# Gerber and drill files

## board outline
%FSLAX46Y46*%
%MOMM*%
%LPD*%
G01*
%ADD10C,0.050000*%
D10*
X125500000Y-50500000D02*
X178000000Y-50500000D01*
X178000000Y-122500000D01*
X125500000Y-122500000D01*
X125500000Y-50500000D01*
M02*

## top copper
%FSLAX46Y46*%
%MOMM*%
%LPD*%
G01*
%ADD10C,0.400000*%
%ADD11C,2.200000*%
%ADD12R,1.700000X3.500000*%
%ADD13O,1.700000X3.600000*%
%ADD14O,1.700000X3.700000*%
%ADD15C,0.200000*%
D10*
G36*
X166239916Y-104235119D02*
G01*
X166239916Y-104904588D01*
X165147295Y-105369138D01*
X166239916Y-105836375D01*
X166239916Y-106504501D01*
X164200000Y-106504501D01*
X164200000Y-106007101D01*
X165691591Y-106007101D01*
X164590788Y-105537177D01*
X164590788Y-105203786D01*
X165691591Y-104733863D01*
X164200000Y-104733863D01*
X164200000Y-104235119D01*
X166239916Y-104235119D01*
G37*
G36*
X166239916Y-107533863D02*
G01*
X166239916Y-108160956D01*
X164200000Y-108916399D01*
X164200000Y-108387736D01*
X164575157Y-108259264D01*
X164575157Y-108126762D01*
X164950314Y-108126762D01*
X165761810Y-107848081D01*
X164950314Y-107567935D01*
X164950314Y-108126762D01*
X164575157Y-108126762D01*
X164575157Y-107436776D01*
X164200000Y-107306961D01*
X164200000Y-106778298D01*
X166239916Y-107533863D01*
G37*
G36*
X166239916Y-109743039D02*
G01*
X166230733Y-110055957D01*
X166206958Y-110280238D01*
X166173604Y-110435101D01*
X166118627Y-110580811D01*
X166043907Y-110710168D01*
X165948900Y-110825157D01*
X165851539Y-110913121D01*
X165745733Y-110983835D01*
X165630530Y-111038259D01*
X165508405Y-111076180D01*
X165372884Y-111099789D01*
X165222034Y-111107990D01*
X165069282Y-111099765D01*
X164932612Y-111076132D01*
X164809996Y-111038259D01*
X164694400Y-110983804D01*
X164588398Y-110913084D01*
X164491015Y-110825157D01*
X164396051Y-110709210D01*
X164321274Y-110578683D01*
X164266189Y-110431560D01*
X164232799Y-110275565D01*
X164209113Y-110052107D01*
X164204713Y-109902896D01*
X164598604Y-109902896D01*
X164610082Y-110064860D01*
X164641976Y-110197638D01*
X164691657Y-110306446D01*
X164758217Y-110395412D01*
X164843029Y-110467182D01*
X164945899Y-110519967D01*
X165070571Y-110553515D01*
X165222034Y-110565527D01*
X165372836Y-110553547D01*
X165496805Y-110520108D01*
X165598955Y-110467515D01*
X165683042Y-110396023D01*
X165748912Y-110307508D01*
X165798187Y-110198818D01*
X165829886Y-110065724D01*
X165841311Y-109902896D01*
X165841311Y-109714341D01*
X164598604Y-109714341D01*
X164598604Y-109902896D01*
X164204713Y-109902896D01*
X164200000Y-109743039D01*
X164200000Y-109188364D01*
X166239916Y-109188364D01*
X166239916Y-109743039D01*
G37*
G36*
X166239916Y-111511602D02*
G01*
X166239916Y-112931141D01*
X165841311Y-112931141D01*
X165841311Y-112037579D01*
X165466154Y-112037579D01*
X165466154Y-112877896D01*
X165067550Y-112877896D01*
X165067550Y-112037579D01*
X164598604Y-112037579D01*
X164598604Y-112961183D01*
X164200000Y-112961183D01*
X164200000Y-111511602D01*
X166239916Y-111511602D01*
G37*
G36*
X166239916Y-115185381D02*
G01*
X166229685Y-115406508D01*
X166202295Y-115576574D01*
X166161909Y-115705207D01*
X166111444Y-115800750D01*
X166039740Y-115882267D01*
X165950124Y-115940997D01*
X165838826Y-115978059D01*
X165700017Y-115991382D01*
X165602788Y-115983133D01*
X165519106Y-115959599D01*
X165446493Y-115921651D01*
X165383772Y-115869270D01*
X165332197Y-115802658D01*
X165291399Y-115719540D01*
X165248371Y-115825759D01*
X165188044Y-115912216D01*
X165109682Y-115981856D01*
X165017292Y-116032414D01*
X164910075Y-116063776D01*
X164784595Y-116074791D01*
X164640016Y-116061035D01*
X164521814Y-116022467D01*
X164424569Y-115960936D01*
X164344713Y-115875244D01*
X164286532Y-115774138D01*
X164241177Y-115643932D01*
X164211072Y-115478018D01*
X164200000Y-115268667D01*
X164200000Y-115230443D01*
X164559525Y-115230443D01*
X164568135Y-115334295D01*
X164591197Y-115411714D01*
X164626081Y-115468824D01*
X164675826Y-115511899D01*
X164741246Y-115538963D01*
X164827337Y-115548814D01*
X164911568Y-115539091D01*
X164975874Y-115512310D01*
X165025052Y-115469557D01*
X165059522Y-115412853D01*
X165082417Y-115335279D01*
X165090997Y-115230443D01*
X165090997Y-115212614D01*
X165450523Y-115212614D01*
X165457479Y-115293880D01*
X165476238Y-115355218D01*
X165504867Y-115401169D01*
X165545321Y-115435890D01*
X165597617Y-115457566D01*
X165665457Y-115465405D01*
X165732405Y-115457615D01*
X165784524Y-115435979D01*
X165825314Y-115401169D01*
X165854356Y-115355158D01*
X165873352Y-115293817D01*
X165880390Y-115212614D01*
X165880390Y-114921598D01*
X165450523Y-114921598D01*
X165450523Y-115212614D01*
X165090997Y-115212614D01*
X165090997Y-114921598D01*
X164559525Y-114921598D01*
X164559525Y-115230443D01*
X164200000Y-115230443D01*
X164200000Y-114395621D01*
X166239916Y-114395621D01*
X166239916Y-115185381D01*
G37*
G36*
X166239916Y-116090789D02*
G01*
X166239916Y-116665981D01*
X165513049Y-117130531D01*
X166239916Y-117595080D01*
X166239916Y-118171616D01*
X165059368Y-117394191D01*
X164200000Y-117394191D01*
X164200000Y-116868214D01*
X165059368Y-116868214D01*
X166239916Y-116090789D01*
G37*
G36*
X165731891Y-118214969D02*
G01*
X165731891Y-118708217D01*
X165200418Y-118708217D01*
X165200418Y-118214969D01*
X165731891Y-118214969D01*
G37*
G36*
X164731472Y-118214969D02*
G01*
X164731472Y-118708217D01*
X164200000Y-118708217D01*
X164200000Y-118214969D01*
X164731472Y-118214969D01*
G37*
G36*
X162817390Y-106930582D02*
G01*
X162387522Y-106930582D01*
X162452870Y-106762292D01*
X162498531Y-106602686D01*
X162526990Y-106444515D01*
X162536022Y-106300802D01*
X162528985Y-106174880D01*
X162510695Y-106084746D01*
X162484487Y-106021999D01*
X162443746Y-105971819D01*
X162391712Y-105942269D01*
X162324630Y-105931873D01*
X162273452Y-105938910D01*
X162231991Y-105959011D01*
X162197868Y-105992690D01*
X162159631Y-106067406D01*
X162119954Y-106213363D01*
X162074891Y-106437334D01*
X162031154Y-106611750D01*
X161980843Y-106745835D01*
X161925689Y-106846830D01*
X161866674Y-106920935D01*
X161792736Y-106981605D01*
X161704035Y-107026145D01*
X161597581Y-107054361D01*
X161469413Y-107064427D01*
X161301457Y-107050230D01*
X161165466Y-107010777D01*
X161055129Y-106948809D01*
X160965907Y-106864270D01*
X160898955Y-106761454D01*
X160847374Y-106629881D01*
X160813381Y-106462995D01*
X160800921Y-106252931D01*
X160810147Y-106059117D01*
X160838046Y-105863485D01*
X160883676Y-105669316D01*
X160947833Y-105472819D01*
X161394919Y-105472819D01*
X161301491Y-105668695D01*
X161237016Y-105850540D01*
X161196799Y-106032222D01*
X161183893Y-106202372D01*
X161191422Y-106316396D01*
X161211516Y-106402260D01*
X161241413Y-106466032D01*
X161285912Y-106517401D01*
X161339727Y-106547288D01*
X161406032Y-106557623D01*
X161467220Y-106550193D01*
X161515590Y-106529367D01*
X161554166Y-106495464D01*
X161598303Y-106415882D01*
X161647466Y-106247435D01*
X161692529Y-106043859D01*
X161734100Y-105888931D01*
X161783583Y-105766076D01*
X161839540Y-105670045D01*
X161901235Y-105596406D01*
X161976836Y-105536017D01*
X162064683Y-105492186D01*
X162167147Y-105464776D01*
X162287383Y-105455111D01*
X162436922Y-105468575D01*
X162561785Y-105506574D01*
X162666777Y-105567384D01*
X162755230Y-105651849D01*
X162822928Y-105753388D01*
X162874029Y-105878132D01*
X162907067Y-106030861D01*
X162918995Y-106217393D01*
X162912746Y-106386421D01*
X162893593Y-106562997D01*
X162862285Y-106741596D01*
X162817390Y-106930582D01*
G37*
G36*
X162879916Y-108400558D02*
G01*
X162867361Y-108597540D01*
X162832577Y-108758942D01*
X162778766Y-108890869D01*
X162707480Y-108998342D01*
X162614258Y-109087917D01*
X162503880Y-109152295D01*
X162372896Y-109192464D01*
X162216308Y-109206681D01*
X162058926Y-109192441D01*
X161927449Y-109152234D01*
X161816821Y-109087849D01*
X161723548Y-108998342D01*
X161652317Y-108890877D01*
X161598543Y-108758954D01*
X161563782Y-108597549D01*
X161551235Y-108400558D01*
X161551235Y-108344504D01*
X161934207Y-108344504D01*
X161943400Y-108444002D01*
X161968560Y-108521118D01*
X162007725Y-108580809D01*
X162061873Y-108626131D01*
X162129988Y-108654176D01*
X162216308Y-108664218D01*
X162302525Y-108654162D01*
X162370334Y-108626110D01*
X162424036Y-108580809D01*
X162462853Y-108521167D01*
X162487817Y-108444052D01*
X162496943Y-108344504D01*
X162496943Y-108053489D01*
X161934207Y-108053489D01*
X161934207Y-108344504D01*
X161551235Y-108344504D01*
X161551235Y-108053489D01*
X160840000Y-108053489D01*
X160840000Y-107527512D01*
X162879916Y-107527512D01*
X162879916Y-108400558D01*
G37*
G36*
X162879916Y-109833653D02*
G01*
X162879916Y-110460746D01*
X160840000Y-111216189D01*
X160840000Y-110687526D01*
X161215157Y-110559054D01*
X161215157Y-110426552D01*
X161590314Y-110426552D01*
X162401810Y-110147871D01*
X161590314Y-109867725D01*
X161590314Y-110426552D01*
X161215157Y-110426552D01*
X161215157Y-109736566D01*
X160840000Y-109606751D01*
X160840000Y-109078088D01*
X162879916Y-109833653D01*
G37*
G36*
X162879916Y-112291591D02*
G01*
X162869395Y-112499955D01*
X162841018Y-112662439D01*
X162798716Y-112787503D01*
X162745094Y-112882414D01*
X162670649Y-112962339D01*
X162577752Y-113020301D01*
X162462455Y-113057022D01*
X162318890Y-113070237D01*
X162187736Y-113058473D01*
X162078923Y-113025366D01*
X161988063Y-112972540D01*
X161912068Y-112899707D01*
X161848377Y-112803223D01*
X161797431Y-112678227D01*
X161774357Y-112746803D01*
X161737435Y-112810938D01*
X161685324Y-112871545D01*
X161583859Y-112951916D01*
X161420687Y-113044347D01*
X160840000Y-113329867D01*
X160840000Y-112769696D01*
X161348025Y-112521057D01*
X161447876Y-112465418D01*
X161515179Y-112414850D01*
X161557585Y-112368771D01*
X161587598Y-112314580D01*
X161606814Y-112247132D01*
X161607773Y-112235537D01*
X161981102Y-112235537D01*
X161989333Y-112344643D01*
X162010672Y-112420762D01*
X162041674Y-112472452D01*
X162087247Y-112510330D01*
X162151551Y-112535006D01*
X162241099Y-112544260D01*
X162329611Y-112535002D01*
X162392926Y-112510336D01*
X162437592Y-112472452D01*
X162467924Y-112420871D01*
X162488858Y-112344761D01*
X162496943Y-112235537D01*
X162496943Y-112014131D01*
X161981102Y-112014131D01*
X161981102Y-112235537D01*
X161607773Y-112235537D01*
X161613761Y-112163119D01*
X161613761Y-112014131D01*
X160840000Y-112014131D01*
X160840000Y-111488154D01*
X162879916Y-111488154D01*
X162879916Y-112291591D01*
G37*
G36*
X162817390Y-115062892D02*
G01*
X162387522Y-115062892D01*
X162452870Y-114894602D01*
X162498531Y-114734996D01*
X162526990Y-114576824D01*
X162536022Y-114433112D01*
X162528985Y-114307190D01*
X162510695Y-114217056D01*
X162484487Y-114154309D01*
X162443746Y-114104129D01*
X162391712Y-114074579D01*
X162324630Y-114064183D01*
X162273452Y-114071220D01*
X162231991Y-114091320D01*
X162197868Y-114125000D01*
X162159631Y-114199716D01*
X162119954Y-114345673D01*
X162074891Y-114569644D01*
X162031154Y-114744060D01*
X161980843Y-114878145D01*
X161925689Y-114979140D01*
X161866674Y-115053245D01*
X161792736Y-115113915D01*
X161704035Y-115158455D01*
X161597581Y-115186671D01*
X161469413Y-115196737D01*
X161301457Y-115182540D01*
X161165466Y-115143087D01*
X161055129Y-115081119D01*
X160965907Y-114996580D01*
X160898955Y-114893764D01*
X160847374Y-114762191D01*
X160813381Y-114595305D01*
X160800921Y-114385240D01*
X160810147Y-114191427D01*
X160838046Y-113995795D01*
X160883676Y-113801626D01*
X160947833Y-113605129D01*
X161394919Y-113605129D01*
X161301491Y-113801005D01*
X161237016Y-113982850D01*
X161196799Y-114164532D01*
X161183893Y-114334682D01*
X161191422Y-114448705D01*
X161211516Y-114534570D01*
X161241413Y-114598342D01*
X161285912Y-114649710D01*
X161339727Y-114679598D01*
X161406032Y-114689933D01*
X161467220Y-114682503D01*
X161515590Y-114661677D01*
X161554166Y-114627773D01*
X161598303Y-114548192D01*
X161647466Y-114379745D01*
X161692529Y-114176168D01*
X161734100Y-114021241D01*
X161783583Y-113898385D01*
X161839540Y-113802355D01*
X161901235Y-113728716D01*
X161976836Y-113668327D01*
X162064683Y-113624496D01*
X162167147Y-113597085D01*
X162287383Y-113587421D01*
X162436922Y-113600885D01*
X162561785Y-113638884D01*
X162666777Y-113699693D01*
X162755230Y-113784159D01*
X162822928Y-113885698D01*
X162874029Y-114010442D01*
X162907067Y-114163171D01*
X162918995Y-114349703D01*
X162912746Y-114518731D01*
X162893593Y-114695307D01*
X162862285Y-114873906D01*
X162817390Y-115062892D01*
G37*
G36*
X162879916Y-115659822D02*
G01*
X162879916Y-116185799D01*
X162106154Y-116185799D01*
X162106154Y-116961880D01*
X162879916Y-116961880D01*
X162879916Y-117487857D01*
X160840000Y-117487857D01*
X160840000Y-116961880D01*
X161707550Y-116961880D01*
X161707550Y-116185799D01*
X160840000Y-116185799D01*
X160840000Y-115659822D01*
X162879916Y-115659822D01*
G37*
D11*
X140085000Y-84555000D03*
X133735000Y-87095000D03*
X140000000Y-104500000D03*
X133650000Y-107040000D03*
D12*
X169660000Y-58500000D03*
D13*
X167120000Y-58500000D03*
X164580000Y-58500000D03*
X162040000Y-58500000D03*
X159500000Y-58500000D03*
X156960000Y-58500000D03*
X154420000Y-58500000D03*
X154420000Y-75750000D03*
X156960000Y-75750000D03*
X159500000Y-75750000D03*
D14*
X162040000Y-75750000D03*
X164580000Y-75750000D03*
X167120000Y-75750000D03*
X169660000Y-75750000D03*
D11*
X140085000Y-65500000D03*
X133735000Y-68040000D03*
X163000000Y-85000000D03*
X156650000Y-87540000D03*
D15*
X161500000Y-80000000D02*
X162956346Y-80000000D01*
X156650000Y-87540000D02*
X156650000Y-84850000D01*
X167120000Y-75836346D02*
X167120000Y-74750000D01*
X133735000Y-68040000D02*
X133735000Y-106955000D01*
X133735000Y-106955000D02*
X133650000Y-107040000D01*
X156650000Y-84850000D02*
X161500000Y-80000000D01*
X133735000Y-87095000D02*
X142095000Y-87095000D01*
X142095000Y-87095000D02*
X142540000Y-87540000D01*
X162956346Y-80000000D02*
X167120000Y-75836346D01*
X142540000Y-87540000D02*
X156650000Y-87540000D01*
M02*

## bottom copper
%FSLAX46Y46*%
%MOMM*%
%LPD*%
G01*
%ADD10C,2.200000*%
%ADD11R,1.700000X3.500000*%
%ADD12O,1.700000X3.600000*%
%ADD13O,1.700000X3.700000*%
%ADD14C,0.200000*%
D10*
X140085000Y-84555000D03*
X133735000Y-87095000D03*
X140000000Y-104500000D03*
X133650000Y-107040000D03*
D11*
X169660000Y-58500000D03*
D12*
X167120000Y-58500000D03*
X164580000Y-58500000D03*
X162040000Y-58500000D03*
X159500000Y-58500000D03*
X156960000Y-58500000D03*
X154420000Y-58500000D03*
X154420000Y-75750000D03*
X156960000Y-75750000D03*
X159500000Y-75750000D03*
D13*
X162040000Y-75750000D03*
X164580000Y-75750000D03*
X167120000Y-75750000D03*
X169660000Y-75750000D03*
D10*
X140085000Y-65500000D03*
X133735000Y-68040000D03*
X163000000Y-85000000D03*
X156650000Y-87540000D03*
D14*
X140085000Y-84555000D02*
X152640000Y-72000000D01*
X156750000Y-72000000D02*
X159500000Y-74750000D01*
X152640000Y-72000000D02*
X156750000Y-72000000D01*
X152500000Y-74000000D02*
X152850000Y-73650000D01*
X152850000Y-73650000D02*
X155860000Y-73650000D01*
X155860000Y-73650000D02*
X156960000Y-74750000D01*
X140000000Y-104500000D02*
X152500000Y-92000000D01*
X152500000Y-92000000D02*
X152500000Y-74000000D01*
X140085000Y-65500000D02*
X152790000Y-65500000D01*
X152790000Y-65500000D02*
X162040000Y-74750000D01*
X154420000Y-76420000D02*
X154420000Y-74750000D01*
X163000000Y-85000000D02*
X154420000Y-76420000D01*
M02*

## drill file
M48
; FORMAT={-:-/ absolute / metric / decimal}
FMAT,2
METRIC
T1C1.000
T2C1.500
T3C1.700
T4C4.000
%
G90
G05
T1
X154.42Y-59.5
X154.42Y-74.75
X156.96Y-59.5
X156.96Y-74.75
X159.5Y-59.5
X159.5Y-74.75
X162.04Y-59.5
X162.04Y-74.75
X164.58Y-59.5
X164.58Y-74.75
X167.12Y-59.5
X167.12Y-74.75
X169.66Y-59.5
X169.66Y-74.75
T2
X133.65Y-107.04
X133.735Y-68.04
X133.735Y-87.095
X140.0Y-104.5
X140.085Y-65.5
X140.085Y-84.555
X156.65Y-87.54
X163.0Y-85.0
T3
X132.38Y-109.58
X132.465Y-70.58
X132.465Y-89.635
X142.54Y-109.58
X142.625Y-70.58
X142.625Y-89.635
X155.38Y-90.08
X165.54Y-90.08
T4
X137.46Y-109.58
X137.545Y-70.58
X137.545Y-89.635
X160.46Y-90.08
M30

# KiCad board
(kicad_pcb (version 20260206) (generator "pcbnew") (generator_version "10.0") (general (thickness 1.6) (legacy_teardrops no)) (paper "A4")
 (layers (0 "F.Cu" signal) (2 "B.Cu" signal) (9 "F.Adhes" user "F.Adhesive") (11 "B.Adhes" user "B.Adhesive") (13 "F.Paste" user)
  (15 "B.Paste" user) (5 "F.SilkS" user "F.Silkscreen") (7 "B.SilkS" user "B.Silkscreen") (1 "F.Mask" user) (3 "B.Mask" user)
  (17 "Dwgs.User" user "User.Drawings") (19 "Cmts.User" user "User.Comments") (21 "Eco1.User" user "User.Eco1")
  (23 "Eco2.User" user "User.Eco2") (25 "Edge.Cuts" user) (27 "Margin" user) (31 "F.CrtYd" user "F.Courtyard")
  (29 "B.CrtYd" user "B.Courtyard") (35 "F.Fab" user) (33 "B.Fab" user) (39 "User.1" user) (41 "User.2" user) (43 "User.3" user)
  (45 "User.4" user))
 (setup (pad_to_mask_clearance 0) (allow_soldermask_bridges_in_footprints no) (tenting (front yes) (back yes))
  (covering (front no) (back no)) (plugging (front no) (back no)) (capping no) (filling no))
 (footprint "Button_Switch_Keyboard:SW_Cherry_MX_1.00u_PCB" (layer "F.Cu") (at 140.085 84.555)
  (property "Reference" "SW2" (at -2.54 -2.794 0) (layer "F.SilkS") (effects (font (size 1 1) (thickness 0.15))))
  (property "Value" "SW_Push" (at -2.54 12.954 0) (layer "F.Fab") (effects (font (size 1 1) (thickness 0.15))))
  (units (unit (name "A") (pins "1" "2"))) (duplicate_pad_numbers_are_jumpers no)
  (pad "" np_thru_hole circle (at -7.62 5.08) (size 1.7 1.7) (drill 1.7) (layers "*.Cu" "*.Mask"))
  (pad "" np_thru_hole circle (at -2.54 5.08) (size 4 4) (drill 4) (layers "*.Cu" "*.Mask"))
  (pad "" np_thru_hole circle (at 2.54 5.08) (size 1.7 1.7) (drill 1.7) (layers "*.Cu" "*.Mask"))
  (pad "1" thru_hole circle (at 0 0) (size 2.2 2.2) (drill 1.5) (layers "*.Cu" "*.Mask") (remove_unused_layers no)
   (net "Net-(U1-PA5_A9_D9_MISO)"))
  (pad "2" thru_hole circle (at -6.35 2.54) (size 2.2 2.2) (drill 1.5) (layers "*.Cu" "*.Mask") (remove_unused_layers no) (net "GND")))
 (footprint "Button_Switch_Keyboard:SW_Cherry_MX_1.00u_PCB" (layer "F.Cu") (at 140 104.5)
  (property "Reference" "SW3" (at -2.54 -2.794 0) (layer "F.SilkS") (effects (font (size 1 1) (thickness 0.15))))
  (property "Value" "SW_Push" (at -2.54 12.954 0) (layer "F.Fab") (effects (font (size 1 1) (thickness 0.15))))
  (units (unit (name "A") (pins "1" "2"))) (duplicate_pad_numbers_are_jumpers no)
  (pad "" np_thru_hole circle (at -7.62 5.08) (size 1.7 1.7) (drill 1.7) (layers "*.Cu" "*.Mask"))
  (pad "" np_thru_hole circle (at -2.54 5.08) (size 4 4) (drill 4) (layers "*.Cu" "*.Mask"))
  (pad "" np_thru_hole circle (at 2.54 5.08) (size 1.7 1.7) (drill 1.7) (layers "*.Cu" "*.Mask"))
  (pad "1" thru_hole circle (at 0 0) (size 2.2 2.2) (drill 1.5) (layers "*.Cu" "*.Mask") (remove_unused_layers no)
   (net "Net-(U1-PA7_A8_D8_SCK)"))
  (pad "2" thru_hole circle (at -6.35 2.54) (size 2.2 2.2) (drill 1.5) (layers "*.Cu" "*.Mask") (remove_unused_layers no) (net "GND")))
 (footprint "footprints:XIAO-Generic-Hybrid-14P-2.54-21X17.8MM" (layer "F.Cu") (at 162.04 67.125 -90)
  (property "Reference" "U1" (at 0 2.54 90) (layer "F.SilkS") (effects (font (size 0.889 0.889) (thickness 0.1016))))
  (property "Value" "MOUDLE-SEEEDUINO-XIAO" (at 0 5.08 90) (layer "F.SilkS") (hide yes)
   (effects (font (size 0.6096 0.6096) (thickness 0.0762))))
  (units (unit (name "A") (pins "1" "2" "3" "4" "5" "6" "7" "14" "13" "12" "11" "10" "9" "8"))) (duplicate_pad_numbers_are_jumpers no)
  (pad "1" thru_hole rect (at -7.625 -7.62 270) (size 3.5 1.7) (drill 1 (offset -1 0)) (layers "*.Cu" "*.Mask") (remove_unused_layers no)
   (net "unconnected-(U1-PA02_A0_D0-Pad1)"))
  (pad "2" thru_hole oval (at -7.625 -5.08 270) (size 3.6 1.7) (drill 1 (offset -1 0)) (layers "*.Cu" "*.Mask") (remove_unused_layers no)
   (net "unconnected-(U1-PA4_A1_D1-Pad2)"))
  (pad "3" thru_hole oval (at -7.625 -2.54 270) (size 3.6 1.7) (drill 1 (offset -1 0)) (layers "*.Cu" "*.Mask") (remove_unused_layers no)
   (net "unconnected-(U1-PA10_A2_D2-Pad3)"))
  (pad "4" thru_hole oval (at -7.625 0 270) (size 3.6 1.7) (drill 1 (offset -1 0)) (layers "*.Cu" "*.Mask") (remove_unused_layers no)
   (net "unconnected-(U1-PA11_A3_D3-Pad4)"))
  (pad "5" thru_hole oval (at -7.625 2.54 270) (size 3.6 1.7) (drill 1 (offset -1 0)) (layers "*.Cu" "*.Mask") (remove_unused_layers no)
   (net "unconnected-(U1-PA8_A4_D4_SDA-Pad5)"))
  (pad "6" thru_hole oval (at -7.625 5.08 90) (size 3.6 1.7) (drill 1 (offset 1 0)) (layers "*.Cu" "*.Mask") (remove_unused_layers no)
   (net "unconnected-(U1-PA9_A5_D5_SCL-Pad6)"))
  (pad "7" thru_hole oval (at -7.625 7.62 270) (size 3.6 1.7) (drill 1 (offset -1 0)) (layers "*.Cu" "*.Mask") (remove_unused_layers no)
   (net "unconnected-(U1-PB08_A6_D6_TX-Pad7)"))
  (pad "8" thru_hole oval (at 7.625 7.62 270) (size 3.6 1.7) (drill 1 (offset 1 0)) (layers "*.Cu" "*.Mask") (remove_unused_layers no)
   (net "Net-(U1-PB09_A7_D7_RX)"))
  (pad "9" thru_hole oval (at 7.625 5.08 270) (size 3.6 1.7) (drill 1 (offset 1 0)) (layers "*.Cu" "*.Mask") (remove_unused_layers no)
   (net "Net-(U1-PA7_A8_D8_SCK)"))
  (pad "10" thru_hole oval (at 7.625 2.54 270) (size 3.6 1.7) (drill 1 (offset 1 0)) (layers "*.Cu" "*.Mask") (remove_unused_layers no)
   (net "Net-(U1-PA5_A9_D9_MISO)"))
  (pad "11" thru_hole oval (at 7.625 0 270) (size 3.7 1.7) (drill 1 (offset 1 0)) (layers "*.Cu" "*.Mask") (remove_unused_layers no)
   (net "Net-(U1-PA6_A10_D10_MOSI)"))
  (pad "12" thru_hole oval (at 7.625 -2.54 270) (size 3.7 1.7) (drill 1 (offset 1 0)) (layers "*.Cu" "*.Mask") (remove_unused_layers no)
   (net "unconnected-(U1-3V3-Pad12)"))
  (pad "13" thru_hole oval (at 7.625 -5.08 270) (size 3.7 1.7) (drill 1 (offset 1 0)) (layers "*.Cu" "*.Mask") (remove_unused_layers no)
   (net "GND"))
  (pad "14" thru_hole oval (at 7.625 -7.62 270) (size 3.7 1.7) (drill 1 (offset 1 0)) (layers "*.Cu" "*.Mask") (remove_unused_layers no)
   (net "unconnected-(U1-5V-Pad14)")))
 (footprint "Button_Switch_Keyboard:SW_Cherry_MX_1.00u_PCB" (layer "F.Cu") (at 140.085 65.5)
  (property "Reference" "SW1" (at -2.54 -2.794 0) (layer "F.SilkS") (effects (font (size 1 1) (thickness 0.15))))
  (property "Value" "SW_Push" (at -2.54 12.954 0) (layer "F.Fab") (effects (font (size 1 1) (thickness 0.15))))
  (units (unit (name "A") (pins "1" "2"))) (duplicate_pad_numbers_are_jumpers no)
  (pad "" np_thru_hole circle (at -7.62 5.08) (size 1.7 1.7) (drill 1.7) (layers "*.Cu" "*.Mask"))
  (pad "" np_thru_hole circle (at -2.54 5.08) (size 4 4) (drill 4) (layers "*.Cu" "*.Mask"))
  (pad "" np_thru_hole circle (at 2.54 5.08) (size 1.7 1.7) (drill 1.7) (layers "*.Cu" "*.Mask"))
  (pad "1" thru_hole circle (at 0 0) (size 2.2 2.2) (drill 1.5) (layers "*.Cu" "*.Mask") (remove_unused_layers no)
   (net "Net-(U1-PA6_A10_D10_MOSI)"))
  (pad "2" thru_hole circle (at -6.35 2.54) (size 2.2 2.2) (drill 1.5) (layers "*.Cu" "*.Mask") (remove_unused_layers no) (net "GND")))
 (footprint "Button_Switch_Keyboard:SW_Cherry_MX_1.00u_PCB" (layer "F.Cu") (at 163 85)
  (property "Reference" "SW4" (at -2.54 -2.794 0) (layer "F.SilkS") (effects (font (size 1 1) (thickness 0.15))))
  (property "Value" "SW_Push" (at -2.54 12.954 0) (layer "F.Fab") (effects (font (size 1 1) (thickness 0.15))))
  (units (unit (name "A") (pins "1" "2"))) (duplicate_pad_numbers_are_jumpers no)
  (pad "" np_thru_hole circle (at -7.62 5.08) (size 1.7 1.7) (drill 1.7) (layers "*.Cu" "*.Mask"))
  (pad "" np_thru_hole circle (at -2.54 5.08) (size 4 4) (drill 4) (layers "*.Cu" "*.Mask"))
  (pad "" np_thru_hole circle (at 2.54 5.08) (size 1.7 1.7) (drill 1.7) (layers "*.Cu" "*.Mask"))
  (pad "1" thru_hole circle (at 0 0) (size 2.2 2.2) (drill 1.5) (layers "*.Cu" "*.Mask") (remove_unused_layers no)
   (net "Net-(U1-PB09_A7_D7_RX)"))
  (pad "2" thru_hole circle (at -6.35 2.54) (size 2.2 2.2) (drill 1.5) (layers "*.Cu" "*.Mask") (remove_unused_layers no) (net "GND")))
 (gr_rect (start 125.5 50.5) (end 178 122.5) (stroke (width 0.05) (type default)) (fill no) (layer "Edge.Cuts"))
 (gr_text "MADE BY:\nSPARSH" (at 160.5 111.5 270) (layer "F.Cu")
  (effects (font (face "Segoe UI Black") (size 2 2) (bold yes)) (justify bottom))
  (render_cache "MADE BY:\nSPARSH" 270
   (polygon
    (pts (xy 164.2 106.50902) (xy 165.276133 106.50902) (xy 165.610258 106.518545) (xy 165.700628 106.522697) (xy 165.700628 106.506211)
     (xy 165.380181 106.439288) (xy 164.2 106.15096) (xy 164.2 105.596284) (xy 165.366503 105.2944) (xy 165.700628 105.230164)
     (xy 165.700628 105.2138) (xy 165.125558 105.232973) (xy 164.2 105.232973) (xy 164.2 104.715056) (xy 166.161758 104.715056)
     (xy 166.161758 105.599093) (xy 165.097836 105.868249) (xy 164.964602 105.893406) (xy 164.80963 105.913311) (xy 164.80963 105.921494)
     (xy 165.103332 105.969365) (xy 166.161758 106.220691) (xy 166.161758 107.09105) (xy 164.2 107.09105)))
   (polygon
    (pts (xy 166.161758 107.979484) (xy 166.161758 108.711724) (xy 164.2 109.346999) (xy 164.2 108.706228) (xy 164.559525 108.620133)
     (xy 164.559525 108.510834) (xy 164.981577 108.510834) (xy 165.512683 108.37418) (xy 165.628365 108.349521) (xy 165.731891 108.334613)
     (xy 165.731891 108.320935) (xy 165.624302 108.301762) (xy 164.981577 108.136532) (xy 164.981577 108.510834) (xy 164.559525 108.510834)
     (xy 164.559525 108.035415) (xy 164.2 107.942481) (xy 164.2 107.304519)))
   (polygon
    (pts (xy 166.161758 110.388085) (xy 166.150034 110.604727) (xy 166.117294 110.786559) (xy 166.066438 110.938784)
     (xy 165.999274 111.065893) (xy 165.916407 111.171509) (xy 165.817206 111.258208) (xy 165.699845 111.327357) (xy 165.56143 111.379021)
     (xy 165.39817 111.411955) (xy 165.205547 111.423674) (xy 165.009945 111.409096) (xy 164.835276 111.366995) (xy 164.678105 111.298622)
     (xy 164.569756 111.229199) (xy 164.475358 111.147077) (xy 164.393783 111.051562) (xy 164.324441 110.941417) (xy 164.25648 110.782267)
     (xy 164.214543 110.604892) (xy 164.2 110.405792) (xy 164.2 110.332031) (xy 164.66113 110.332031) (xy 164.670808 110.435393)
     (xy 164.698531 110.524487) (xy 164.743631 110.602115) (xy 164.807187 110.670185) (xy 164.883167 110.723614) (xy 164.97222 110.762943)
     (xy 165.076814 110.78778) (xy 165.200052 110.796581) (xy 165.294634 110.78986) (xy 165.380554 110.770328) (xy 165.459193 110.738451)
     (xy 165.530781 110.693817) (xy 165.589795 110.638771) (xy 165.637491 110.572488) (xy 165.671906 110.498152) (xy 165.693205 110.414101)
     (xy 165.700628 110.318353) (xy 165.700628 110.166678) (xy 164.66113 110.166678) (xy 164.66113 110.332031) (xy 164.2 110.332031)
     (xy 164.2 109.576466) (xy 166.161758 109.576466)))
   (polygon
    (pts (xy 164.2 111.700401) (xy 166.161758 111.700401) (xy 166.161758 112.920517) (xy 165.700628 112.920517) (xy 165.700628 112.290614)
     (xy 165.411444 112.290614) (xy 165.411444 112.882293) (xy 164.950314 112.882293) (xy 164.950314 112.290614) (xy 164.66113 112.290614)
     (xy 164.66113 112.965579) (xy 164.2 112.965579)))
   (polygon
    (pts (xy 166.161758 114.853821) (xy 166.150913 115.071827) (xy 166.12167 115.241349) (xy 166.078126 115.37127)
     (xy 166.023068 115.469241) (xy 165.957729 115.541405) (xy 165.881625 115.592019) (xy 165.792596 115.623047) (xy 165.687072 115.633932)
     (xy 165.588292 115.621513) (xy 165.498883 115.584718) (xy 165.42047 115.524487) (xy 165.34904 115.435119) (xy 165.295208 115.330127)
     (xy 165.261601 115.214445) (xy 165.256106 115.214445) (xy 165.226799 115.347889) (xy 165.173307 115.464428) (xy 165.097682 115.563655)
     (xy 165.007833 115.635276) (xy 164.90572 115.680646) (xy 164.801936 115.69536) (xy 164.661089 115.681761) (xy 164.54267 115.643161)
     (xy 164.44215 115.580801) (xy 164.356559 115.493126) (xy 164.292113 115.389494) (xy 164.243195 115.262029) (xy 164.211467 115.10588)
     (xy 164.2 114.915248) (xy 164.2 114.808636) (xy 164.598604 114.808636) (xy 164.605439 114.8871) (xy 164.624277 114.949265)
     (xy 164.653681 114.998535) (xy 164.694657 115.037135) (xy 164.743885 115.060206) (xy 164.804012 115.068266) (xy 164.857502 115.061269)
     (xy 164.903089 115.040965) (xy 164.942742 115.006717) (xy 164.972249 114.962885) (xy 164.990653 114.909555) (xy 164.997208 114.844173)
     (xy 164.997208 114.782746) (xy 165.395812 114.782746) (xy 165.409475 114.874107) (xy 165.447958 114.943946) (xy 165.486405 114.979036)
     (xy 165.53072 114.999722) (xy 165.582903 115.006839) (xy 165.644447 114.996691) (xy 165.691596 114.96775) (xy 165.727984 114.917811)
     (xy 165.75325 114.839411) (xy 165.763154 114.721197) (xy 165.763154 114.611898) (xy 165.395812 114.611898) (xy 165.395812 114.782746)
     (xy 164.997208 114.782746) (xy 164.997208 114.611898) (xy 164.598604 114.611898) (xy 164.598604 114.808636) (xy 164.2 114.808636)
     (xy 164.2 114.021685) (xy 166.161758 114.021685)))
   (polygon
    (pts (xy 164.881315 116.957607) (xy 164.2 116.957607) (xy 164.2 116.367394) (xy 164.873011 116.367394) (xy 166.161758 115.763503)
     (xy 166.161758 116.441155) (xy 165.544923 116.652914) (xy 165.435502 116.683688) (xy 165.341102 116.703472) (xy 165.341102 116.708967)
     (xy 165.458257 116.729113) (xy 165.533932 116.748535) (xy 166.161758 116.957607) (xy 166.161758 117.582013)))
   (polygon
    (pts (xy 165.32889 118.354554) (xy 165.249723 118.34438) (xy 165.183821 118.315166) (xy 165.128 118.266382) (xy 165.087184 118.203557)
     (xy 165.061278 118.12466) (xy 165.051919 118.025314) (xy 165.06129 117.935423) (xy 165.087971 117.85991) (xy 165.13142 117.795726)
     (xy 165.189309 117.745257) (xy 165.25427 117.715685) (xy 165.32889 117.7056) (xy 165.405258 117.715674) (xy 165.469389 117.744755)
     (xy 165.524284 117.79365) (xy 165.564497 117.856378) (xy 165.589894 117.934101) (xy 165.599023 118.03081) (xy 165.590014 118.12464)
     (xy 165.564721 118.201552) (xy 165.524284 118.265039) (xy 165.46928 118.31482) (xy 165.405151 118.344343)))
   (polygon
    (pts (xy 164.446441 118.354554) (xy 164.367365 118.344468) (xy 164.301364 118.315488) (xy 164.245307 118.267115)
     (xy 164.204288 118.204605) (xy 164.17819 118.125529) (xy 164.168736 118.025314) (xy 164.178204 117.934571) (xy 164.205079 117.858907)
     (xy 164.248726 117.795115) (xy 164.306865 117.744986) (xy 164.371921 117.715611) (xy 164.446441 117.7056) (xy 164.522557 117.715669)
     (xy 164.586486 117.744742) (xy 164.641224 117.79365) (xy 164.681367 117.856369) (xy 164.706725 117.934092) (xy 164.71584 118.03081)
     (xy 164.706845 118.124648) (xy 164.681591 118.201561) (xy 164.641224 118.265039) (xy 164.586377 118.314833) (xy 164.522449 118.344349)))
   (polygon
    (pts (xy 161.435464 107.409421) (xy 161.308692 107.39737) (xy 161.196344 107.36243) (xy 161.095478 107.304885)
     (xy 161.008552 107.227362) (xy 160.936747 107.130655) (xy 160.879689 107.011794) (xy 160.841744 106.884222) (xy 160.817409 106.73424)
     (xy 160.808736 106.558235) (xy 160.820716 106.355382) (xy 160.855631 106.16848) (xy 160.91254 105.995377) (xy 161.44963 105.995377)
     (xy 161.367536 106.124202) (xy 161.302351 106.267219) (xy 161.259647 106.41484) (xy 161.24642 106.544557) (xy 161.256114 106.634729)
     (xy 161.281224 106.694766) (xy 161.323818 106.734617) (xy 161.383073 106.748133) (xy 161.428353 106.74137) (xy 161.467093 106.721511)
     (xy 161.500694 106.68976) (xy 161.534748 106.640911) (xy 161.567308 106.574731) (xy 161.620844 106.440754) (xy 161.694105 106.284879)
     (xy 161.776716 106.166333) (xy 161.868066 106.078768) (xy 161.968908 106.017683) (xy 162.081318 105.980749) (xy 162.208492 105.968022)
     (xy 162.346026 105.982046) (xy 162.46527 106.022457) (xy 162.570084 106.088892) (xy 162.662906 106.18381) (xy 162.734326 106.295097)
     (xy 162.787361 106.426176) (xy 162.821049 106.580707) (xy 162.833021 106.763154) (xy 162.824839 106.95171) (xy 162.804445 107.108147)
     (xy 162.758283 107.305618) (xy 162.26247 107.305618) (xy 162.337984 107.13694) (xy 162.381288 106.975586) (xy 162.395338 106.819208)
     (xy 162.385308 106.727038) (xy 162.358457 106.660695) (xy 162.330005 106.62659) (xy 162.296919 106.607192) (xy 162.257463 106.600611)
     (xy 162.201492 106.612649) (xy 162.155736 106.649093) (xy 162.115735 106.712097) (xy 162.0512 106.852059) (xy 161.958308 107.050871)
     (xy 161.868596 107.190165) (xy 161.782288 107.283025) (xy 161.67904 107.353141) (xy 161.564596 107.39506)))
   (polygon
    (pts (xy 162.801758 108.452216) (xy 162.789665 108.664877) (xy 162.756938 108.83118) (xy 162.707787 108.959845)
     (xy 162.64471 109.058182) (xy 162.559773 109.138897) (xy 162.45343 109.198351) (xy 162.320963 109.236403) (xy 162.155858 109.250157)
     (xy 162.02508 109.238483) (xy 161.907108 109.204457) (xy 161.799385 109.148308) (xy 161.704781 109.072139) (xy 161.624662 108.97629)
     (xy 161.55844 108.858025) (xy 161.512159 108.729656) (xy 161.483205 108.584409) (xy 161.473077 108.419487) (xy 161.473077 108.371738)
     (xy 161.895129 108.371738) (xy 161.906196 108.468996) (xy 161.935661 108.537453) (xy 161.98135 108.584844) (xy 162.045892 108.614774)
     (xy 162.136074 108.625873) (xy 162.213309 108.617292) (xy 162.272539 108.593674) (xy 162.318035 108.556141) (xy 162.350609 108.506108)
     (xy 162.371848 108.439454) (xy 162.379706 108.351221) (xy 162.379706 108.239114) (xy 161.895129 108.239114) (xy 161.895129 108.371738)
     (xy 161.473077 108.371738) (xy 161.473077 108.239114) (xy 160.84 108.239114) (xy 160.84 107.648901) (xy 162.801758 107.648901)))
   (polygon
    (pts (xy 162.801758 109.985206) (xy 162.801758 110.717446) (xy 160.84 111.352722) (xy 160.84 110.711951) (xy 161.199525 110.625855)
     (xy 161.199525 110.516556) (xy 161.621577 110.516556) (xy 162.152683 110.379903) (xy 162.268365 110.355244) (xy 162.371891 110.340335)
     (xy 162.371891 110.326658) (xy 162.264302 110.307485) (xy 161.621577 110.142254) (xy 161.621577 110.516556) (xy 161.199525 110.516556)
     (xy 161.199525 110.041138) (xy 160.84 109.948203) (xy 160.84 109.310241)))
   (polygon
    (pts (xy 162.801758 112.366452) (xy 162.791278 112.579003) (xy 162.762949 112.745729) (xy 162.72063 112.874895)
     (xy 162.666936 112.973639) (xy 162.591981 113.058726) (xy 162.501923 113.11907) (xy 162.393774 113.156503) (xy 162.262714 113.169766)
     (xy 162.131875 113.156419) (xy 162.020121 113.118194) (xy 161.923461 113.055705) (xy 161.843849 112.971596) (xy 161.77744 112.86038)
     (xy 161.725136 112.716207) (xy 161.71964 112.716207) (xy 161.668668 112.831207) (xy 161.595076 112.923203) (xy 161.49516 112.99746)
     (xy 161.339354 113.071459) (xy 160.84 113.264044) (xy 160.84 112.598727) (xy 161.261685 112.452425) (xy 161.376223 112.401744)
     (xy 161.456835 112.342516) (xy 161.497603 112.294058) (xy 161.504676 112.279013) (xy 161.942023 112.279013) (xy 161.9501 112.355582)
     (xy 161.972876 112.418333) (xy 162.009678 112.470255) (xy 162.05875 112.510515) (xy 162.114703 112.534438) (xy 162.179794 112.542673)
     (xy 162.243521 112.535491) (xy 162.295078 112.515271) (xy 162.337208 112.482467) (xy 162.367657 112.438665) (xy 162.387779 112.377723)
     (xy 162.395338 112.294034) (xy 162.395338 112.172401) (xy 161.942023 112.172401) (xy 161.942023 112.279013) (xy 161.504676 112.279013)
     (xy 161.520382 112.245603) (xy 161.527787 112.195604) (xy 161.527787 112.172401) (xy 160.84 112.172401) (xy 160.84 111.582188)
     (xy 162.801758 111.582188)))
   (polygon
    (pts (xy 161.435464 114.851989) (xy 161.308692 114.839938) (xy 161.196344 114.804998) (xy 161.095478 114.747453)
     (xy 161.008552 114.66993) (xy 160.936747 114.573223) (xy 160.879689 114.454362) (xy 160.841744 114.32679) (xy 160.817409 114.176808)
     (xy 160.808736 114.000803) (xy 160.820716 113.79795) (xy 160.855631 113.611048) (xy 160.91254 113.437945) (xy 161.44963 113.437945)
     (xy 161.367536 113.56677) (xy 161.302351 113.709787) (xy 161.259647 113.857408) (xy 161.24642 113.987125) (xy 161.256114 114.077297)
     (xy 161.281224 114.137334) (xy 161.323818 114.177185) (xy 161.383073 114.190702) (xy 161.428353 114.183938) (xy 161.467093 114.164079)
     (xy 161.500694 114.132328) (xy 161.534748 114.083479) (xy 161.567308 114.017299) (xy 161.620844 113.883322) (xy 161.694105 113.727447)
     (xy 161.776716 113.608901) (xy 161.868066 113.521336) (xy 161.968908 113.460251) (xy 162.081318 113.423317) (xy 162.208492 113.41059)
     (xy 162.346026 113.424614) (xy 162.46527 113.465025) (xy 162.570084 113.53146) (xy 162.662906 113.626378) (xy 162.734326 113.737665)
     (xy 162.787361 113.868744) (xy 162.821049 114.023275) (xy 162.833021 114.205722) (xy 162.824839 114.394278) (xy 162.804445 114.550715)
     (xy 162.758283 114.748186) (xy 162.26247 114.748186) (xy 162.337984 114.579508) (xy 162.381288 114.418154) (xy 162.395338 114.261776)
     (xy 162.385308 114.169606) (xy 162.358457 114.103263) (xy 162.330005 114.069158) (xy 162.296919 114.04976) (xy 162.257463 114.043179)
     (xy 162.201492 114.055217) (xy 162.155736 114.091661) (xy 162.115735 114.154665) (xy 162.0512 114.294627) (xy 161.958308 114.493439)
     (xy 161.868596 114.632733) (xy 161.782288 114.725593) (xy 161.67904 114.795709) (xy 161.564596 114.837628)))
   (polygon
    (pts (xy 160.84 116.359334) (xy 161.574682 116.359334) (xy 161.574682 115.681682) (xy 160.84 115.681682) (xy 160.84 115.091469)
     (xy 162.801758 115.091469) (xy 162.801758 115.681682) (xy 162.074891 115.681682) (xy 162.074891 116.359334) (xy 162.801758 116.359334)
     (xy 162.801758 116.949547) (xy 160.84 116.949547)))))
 (segment (start 140.085 84.555) (end 152.64 72) (width 0.2) (layer "B.Cu") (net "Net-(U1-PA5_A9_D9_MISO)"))
 (segment (start 156.75 72) (end 159.5 74.75) (width 0.2) (layer "B.Cu") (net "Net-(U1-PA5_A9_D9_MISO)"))
 (segment (start 152.64 72) (end 156.75 72) (width 0.2) (layer "B.Cu") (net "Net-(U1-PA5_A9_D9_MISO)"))
 (segment (start 161.5 80) (end 162.956346 80) (width 0.2) (layer "F.Cu") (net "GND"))
 (segment (start 156.65 87.54) (end 156.65 84.85) (width 0.2) (layer "F.Cu") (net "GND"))
 (segment (start 167.12 75.836346) (end 167.12 74.75) (width 0.2) (layer "F.Cu") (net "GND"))
 (segment (start 133.735 68.04) (end 133.735 106.955) (width 0.2) (layer "F.Cu") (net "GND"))
 (segment (start 133.735 106.955) (end 133.65 107.04) (width 0.2) (layer "F.Cu") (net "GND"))
 (segment (start 156.65 84.85) (end 161.5 80) (width 0.2) (layer "F.Cu") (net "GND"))
 (segment (start 133.735 87.095) (end 142.095 87.095) (width 0.2) (layer "F.Cu") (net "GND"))
 (segment (start 142.095 87.095) (end 142.54 87.54) (width 0.2) (layer "F.Cu") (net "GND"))
 (segment (start 162.956346 80) (end 167.12 75.836346) (width 0.2) (layer "F.Cu") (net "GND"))
 (segment (start 142.54 87.54) (end 156.65 87.54) (width 0.2) (layer "F.Cu") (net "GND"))
 (segment (start 152.5 74) (end 152.85 73.65) (width 0.2) (layer "B.Cu") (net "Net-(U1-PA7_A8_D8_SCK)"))
 (segment (start 152.85 73.65) (end 155.86 73.65) (width 0.2) (layer "B.Cu") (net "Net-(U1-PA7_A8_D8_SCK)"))
 (segment (start 155.86 73.65) (end 156.96 74.75) (width 0.2) (layer "B.Cu") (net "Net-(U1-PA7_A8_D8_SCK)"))
 (segment (start 140 104.5) (end 152.5 92) (width 0.2) (layer "B.Cu") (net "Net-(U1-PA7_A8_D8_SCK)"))
 (segment (start 152.5 92) (end 152.5 74) (width 0.2) (layer "B.Cu") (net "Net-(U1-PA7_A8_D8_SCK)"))
 (segment (start 140.085 65.5) (end 152.79 65.5) (width 0.2) (layer "B.Cu") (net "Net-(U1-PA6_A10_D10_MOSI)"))
 (segment (start 152.79 65.5) (end 162.04 74.75) (width 0.2) (layer "B.Cu") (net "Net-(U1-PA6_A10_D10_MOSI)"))
 (segment (start 154.42 76.42) (end 154.42 74.75) (width 0.2) (layer "B.Cu") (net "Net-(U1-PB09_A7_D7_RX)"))
 (segment (start 163 85) (end 154.42 76.42) (width 0.2) (layer "B.Cu") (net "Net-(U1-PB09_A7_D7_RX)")))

